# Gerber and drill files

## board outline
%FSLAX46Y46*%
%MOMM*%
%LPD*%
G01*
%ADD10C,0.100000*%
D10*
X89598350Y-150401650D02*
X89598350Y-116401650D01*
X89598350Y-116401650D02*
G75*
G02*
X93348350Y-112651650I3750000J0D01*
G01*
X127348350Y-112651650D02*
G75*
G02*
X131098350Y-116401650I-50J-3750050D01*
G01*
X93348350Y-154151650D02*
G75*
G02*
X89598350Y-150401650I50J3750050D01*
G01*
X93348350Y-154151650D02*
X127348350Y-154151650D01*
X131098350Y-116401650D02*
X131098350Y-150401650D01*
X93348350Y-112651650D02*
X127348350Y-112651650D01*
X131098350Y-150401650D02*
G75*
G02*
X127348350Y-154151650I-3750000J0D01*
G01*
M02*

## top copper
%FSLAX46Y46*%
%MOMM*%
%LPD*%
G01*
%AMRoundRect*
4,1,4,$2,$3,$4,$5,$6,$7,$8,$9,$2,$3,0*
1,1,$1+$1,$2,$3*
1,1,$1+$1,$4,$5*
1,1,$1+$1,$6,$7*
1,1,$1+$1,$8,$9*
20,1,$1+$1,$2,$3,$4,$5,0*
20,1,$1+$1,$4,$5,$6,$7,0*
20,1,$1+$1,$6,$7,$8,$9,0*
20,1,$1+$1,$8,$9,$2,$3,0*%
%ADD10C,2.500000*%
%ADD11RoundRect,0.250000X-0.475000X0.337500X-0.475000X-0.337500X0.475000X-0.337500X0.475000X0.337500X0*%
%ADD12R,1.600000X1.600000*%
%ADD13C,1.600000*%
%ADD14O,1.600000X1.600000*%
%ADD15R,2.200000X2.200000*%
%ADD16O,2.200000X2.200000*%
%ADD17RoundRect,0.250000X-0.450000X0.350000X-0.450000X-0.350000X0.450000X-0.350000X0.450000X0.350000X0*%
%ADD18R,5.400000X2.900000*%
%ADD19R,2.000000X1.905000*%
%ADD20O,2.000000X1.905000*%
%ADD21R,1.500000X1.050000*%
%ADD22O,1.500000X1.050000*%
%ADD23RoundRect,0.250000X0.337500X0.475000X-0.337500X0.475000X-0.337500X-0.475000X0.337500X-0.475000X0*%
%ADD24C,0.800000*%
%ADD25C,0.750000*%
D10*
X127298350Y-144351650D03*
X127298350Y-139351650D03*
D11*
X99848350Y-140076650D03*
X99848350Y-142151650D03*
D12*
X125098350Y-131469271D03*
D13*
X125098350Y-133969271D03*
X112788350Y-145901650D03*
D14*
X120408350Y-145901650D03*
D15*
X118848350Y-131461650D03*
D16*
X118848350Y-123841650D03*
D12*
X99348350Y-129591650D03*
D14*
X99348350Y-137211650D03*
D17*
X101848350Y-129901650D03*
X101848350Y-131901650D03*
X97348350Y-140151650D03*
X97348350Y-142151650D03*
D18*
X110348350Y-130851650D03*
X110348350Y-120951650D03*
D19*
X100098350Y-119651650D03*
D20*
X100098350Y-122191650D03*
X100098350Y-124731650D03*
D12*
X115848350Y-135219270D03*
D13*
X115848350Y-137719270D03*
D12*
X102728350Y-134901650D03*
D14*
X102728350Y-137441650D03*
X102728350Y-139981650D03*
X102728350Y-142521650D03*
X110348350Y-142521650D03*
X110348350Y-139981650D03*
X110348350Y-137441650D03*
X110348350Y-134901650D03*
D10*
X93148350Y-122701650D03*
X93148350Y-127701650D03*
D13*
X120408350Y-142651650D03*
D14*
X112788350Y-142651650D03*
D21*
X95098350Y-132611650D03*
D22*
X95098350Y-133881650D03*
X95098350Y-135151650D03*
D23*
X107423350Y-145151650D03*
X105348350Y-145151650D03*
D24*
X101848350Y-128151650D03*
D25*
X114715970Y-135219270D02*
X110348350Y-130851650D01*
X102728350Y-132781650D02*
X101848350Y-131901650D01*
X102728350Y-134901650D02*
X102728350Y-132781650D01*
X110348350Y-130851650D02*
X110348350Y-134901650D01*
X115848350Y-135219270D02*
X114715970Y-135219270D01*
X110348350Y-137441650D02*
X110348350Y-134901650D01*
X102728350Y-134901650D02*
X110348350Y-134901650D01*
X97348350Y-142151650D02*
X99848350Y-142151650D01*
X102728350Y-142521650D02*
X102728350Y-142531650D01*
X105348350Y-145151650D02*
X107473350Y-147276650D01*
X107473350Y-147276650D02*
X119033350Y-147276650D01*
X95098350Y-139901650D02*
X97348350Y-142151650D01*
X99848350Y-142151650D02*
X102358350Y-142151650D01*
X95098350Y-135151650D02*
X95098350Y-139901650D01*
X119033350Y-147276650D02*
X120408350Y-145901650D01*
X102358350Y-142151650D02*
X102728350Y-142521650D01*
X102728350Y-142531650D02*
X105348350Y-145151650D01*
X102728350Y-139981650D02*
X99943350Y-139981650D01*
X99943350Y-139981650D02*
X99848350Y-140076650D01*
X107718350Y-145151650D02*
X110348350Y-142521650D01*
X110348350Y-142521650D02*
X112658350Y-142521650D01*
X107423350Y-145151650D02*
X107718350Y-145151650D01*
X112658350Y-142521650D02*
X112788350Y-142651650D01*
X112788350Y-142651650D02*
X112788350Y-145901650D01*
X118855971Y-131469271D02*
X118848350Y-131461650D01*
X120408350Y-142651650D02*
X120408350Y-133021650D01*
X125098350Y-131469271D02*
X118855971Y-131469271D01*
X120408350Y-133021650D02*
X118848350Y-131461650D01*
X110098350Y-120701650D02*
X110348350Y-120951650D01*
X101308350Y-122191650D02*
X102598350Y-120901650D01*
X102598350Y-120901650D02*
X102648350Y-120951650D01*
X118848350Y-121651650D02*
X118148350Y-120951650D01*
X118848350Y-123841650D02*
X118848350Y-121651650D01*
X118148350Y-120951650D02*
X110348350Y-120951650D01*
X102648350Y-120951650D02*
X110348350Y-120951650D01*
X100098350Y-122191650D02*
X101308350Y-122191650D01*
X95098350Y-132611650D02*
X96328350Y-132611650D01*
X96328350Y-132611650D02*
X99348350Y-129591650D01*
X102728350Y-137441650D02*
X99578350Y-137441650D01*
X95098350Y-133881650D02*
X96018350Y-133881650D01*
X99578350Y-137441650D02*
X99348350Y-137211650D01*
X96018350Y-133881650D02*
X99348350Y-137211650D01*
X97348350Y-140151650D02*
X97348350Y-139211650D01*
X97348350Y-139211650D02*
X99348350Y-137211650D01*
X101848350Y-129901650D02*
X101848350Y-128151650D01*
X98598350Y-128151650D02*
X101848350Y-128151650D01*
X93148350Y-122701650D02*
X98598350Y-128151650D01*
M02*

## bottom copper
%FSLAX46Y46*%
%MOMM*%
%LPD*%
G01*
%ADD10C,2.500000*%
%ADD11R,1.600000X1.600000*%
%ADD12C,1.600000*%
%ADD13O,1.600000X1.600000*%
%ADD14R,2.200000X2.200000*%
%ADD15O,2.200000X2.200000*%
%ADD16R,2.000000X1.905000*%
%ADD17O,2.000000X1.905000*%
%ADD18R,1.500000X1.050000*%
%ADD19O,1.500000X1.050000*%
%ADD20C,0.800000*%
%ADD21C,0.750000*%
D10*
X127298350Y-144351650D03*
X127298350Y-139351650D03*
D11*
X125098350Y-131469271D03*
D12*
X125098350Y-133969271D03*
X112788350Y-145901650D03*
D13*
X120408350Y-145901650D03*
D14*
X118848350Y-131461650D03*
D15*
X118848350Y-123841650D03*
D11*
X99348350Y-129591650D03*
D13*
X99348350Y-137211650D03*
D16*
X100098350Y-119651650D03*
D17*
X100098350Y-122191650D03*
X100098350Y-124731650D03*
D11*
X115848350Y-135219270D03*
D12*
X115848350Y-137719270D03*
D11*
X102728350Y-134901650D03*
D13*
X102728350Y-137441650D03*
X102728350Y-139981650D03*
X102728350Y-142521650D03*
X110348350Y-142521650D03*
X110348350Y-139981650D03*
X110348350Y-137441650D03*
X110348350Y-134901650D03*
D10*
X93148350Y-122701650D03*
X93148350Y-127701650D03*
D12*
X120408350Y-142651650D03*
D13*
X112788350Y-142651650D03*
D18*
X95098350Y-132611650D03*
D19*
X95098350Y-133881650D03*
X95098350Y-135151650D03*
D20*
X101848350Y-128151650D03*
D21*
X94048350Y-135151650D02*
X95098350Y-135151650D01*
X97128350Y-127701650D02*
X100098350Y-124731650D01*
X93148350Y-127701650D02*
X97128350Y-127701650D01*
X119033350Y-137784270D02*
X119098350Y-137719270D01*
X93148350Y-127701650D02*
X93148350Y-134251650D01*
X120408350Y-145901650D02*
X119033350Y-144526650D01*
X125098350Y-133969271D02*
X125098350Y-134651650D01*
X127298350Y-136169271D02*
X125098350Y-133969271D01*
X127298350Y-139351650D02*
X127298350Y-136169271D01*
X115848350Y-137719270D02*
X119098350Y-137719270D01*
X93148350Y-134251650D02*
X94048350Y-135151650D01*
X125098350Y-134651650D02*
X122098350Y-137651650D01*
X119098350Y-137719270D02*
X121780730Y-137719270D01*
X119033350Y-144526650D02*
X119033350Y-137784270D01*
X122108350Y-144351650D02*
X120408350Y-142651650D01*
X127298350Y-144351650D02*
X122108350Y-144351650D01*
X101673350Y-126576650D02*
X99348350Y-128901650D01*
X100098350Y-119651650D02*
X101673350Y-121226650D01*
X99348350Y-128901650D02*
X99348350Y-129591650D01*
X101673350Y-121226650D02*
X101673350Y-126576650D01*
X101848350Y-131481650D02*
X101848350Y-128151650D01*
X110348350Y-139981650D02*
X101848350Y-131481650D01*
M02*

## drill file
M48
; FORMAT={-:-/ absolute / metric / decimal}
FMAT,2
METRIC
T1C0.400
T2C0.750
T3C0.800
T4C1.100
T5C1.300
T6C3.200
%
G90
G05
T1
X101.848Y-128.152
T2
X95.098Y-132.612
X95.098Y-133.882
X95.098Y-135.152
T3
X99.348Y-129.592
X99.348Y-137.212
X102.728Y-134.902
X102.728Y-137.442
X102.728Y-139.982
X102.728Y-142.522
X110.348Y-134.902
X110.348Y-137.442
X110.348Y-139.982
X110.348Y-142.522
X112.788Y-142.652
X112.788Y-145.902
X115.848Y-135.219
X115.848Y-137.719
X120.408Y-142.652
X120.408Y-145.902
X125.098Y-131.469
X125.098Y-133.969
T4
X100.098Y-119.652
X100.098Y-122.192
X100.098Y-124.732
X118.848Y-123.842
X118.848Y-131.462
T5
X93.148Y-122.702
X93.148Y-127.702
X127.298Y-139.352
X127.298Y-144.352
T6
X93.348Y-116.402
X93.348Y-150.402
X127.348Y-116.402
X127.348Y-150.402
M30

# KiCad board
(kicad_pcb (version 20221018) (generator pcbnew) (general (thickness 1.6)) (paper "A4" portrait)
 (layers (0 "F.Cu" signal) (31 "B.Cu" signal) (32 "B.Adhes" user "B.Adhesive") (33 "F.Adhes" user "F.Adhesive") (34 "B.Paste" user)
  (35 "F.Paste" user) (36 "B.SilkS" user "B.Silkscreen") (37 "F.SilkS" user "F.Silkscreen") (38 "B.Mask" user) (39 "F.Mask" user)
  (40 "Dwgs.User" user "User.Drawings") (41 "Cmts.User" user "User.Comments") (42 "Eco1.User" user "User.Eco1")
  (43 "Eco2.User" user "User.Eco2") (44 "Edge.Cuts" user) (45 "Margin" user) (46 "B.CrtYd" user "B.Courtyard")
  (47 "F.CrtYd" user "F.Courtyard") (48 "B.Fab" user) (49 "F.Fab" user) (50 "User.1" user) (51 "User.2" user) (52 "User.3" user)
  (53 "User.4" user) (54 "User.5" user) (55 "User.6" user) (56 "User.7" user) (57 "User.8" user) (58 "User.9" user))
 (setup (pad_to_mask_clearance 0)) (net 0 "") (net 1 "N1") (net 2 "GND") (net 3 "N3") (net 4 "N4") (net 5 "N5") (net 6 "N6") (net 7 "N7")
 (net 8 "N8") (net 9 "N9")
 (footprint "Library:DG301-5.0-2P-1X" (layer "F.Cu") (at 127.29835 141.85165 90)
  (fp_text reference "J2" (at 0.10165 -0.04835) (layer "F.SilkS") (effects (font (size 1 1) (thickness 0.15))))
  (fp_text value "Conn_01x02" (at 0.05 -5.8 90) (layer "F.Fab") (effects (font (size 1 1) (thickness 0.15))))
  (pad "1" thru_hole circle (at -2.5 0 90) (size 2.5 2.5) (drill 1.3) (layers "*.Cu" "*.Mask") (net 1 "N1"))
  (pad "2" thru_hole circle (at 2.5 0 90) (size 2.5 2.5) (drill 1.3) (layers "*.Cu" "*.Mask") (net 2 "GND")))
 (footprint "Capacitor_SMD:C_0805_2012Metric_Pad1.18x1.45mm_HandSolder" (layer "F.Cu") (at 99.84835 141.11415 -90)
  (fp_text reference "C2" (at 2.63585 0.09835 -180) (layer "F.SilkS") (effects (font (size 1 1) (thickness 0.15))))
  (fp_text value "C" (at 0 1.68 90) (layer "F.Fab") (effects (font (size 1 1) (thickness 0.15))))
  (pad "1" smd roundrect (at -1.0375 0 270) (size 1.175 1.45) (layers "F.Cu" "F.Paste" "F.Mask") (roundrect_rratio 0.212766) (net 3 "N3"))
  (pad "2" smd roundrect (at 1.0375 0 270) (size 1.175 1.45) (layers "F.Cu" "F.Paste" "F.Mask") (roundrect_rratio 0.212766) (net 2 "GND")))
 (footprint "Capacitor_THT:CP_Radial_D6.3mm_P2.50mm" (layer "F.Cu") (at 125.09835 131.469271 -90)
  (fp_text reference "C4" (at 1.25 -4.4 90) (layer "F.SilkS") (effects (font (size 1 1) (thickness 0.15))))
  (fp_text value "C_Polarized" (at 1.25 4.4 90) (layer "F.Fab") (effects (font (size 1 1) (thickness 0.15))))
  (pad "1" thru_hole rect (at 0 0 270) (size 1.6 1.6) (drill 0.8) (layers "*.Cu" "*.Mask") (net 1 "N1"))
  (pad "2" thru_hole circle (at 2.5 0 270) (size 1.6 1.6) (drill 0.8) (layers "*.Cu" "*.Mask") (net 2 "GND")))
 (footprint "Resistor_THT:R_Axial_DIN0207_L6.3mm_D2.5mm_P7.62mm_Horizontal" (layer "F.Cu") (at 112.78835 145.90165)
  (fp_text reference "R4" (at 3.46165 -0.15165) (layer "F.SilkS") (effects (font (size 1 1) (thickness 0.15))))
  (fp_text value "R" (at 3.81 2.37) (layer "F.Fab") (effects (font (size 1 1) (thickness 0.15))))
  (pad "1" thru_hole circle (at 0 0) (size 1.6 1.6) (drill 0.8) (layers "*.Cu" "*.Mask") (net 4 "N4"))
  (pad "2" thru_hole oval (at 7.62 0) (size 1.6 1.6) (drill 0.8) (layers "*.Cu" "*.Mask") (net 2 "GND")))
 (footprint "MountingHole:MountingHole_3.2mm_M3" (layer "F.Cu") (at 93.34835 116.40165)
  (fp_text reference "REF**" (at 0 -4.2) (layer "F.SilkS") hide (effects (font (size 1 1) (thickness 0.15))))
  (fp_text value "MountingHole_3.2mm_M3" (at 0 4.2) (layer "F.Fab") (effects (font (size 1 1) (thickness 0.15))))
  (pad "" np_thru_hole circle (at 0 0) (size 3.2 3.2) (drill 3.2) (layers "*.Cu" "*.Mask")))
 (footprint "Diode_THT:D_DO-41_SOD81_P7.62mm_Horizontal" (layer "F.Cu") (at 118.84835 131.46165 90)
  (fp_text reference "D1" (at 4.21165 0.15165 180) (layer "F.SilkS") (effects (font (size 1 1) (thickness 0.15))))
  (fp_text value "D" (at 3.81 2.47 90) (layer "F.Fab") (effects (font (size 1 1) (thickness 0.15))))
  (pad "1" thru_hole rect (at 0 0 90) (size 2.2 2.2) (drill 1.1) (layers "*.Cu" "*.Mask") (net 1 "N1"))
  (pad "2" thru_hole oval (at 7.62 0 90) (size 2.2 2.2) (drill 1.1) (layers "*.Cu" "*.Mask") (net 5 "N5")))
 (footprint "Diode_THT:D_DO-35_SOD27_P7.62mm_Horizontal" (layer "F.Cu") (at 99.34835 129.59165 -90)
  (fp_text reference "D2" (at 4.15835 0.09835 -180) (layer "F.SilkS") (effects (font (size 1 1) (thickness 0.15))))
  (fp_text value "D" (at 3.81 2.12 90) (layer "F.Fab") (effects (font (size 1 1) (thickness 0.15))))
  (pad "1" thru_hole rect (at 0 0 270) (size 1.6 1.6) (drill 0.8) (layers "*.Cu" "*.Mask") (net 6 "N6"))
  (pad "2" thru_hole oval (at 7.62 0 270) (size 1.6 1.6) (drill 0.8) (layers "*.Cu" "*.Mask") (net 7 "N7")))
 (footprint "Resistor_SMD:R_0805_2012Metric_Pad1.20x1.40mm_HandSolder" (layer "F.Cu") (at 101.84835 130.90165 -90)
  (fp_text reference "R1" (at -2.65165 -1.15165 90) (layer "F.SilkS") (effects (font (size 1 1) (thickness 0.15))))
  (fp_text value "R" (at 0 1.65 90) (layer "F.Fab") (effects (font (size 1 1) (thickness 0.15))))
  (pad "1" smd roundrect (at -1 0 270) (size 1.2 1.4) (layers "F.Cu" "F.Paste" "F.Mask") (roundrect_rratio 0.208333) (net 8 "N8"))
  (pad "2" smd roundrect (at 1 0 270) (size 1.2 1.4) (layers "F.Cu" "F.Paste" "F.Mask") (roundrect_rratio 0.208333) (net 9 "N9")))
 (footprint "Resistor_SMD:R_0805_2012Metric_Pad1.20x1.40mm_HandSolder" (layer "F.Cu") (at 97.34835 141.15165 -90)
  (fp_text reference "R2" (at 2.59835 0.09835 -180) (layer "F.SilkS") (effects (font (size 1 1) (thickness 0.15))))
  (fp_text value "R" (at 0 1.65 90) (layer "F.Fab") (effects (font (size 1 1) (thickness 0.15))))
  (pad "1" smd roundrect (at -1 0 270) (size 1.2 1.4) (layers "F.Cu" "F.Paste" "F.Mask") (roundrect_rratio 0.208333) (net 7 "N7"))
  (pad "2" smd roundrect (at 1 0 270) (size 1.2 1.4) (layers "F.Cu" "F.Paste" "F.Mask") (roundrect_rratio 0.208333) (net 2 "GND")))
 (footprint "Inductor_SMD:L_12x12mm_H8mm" (layer "F.Cu") (at 110.34835 125.90165 90)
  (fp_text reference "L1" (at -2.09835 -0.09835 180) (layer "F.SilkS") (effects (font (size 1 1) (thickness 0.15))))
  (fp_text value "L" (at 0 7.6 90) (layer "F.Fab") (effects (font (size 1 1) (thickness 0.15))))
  (pad "1" smd rect (at -4.95 0 90) (size 2.9 5.4) (layers "F.Cu" "F.Paste" "F.Mask") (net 9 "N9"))
  (pad "2" smd rect (at 4.95 0 90) (size 2.9 5.4) (layers "F.Cu" "F.Paste" "F.Mask") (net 5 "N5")))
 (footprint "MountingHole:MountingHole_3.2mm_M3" (layer "F.Cu") (at 127.34835 150.40165)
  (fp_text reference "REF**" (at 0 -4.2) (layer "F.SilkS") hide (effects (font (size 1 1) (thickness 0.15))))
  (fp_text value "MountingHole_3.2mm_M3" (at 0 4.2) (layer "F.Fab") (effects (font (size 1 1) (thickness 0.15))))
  (pad "" np_thru_hole circle (at 0 0) (size 3.2 3.2) (drill 3.2) (layers "*.Cu" "*.Mask")))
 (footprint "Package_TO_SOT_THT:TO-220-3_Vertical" (layer "F.Cu") (at 100.09835 119.65165 -90)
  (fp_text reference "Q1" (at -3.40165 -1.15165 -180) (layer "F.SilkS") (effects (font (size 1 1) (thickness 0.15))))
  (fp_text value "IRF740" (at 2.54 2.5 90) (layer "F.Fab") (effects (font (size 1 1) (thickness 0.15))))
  (pad "1" thru_hole rect (at 0 0 270) (size 1.905 2) (drill 1.1) (layers "*.Cu" "*.Mask") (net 6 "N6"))
  (pad "2" thru_hole oval (at 2.54 0 270) (size 1.905 2) (drill 1.1) (layers "*.Cu" "*.Mask") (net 5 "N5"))
  (pad "3" thru_hole oval (at 5.08 0 270) (size 1.905 2) (drill 1.1) (layers "*.Cu" "*.Mask") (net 2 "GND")))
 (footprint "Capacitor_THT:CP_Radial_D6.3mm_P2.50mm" (layer "F.Cu") (at 115.84835 135.21927 -90)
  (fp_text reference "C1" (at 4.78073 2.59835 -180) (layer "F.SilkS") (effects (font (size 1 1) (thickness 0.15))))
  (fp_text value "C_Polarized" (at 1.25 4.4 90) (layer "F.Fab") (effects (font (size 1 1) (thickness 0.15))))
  (pad "1" thru_hole rect (at 0 0 270) (size 1.6 1.6) (drill 0.8) (layers "*.Cu" "*.Mask") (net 9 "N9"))
  (pad "2" thru_hole circle (at 2.5 0 270) (size 1.6 1.6) (drill 0.8) (layers "*.Cu" "*.Mask") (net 2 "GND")))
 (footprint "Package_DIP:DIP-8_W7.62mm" (layer "F.Cu") (at 102.72835 134.90165)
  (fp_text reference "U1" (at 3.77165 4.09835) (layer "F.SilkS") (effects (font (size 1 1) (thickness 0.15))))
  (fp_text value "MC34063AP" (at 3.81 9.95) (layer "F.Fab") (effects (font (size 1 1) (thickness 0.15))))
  (pad "1" thru_hole rect (at 0 0) (size 1.6 1.6) (drill 0.8) (layers "*.Cu" "*.Mask") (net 9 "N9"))
  (pad "2" thru_hole oval (at 0 2.54) (size 1.6 1.6) (drill 0.8) (layers "*.Cu" "*.Mask") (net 7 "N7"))
  (pad "3" thru_hole oval (at 0 5.08) (size 1.6 1.6) (drill 0.8) (layers "*.Cu" "*.Mask") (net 3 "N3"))
  (pad "4" thru_hole oval (at 0 7.62) (size 1.6 1.6) (drill 0.8) (layers "*.Cu" "*.Mask") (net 2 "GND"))
  (pad "5" thru_hole oval (at 7.62 7.62) (size 1.6 1.6) (drill 0.8) (layers "*.Cu" "*.Mask") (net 4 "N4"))
  (pad "6" thru_hole oval (at 7.62 5.08) (size 1.6 1.6) (drill 0.8) (layers "*.Cu" "*.Mask") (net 8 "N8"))
  (pad "7" thru_hole oval (at 7.62 2.54) (size 1.6 1.6) (drill 0.8) (layers "*.Cu" "*.Mask") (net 9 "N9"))
  (pad "8" thru_hole oval (at 7.62 0) (size 1.6 1.6) (drill 0.8) (layers "*.Cu" "*.Mask") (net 9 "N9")))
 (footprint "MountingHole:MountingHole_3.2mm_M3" (layer "F.Cu") (at 93.34835 150.40165)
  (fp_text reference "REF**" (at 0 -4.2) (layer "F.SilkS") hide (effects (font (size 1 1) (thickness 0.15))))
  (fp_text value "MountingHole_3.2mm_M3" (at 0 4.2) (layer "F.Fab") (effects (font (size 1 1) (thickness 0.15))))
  (pad "" np_thru_hole circle (at 0 0) (size 3.2 3.2) (drill 3.2) (layers "*.Cu" "*.Mask")))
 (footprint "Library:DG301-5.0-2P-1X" (layer "F.Cu") (at 93.14835 125.20165 -90)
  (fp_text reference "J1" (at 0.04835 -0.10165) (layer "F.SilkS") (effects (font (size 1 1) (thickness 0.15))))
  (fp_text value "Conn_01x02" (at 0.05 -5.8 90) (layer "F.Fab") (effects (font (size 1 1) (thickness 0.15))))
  (pad "1" thru_hole circle (at -2.5 0 270) (size 2.5 2.5) (drill 1.3) (layers "*.Cu" "*.Mask") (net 8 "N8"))
  (pad "2" thru_hole circle (at 2.5 0 270) (size 2.5 2.5) (drill 1.3) (layers "*.Cu" "*.Mask") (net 2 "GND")))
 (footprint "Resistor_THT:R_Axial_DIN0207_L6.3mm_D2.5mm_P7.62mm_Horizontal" (layer "F.Cu") (at 120.40835 142.65165 180)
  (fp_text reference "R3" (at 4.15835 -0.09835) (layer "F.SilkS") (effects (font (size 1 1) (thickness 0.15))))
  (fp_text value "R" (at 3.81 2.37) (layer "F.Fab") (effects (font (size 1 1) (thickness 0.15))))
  (pad "1" thru_hole circle (at 0 0 180) (size 1.6 1.6) (drill 0.8) (layers "*.Cu" "*.Mask") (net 1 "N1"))
  (pad "2" thru_hole oval (at 7.62 0 180) (size 1.6 1.6) (drill 0.8) (layers "*.Cu" "*.Mask") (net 4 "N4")))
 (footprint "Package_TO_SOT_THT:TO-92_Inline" (layer "F.Cu") (at 95.09835 132.61165 -90)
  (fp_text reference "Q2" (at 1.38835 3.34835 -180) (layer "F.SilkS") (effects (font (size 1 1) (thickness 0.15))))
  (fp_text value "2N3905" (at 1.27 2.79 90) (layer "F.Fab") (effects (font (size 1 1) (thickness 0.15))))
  (pad "1" thru_hole rect (at 0 0 270) (size 1.05 1.5) (drill 0.75) (layers "*.Cu" "*.Mask") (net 6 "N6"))
  (pad "2" thru_hole oval (at 1.27 0 270) (size 1.05 1.5) (drill 0.75) (layers "*.Cu" "*.Mask") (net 7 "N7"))
  (pad "3" thru_hole oval (at 2.54 0 270) (size 1.05 1.5) (drill 0.75) (layers "*.Cu" "*.Mask") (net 2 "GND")))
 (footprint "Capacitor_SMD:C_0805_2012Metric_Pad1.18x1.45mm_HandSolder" (layer "F.Cu") (at 106.38585 145.15165 180)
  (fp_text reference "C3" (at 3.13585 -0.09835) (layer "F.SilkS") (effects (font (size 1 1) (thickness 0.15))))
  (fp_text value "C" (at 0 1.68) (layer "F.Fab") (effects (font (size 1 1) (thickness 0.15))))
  (pad "1" smd roundrect (at -1.0375 0 180) (size 1.175 1.45) (layers "F.Cu" "F.Paste" "F.Mask") (roundrect_rratio 0.212766) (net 4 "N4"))
  (pad "2" smd roundrect (at 1.0375 0 180) (size 1.175 1.45) (layers "F.Cu" "F.Paste" "F.Mask") (roundrect_rratio 0.212766) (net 2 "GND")))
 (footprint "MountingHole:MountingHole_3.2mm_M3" (layer "F.Cu") (at 127.34835 116.40165)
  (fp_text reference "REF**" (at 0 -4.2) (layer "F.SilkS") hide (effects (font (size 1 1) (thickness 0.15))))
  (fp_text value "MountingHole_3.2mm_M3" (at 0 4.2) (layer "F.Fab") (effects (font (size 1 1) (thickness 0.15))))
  (pad "" np_thru_hole circle (at 0 0) (size 3.2 3.2) (drill 3.2) (layers "*.Cu" "*.Mask")))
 (gr_line (start 89.59835 150.40165) (end 89.59835 116.40165) (stroke (width 0.1) (type default)) (layer "Edge.Cuts"))
 (gr_arc (start 89.59835 116.40165) (mid 90.6967 113.75) (end 93.34835 112.65165) (stroke (width 0.1) (type default)) (layer "Edge.Cuts"))
 (gr_arc (start 127.34835 112.65165) (mid 130 113.75) (end 131.09835 116.40165) (stroke (width 0.1) (type default)) (layer "Edge.Cuts"))
 (gr_arc (start 93.34835 154.15165) (mid 90.6967 153.0533) (end 89.59835 150.40165) (stroke (width 0.1) (type default)) (layer "Edge.Cuts"))
 (gr_line (start 93.34835 154.15165) (end 127.34835 154.15165) (stroke (width 0.1) (type default)) (layer "Edge.Cuts"))
 (gr_line (start 131.09835 116.40165) (end 131.09835 150.40165) (stroke (width 0.1) (type default)) (layer "Edge.Cuts"))
 (gr_line (start 93.34835 112.65165) (end 127.34835 112.65165) (stroke (width 0.1) (type default)) (layer "Edge.Cuts"))
 (gr_arc (start 131.09835 150.40165) (mid 130 153.0533) (end 127.34835 154.15165) (stroke (width 0.1) (type default)) (layer "Edge.Cuts"))
 (segment (start 114.71597 135.21927) (end 110.34835 130.85165) (width 0.75) (layer "F.Cu") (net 9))
 (segment (start 102.72835 132.78165) (end 101.84835 131.90165) (width 0.75) (layer "F.Cu") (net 9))
 (segment (start 102.72835 134.90165) (end 102.72835 132.78165) (width 0.75) (layer "F.Cu") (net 9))
 (segment (start 110.34835 130.85165) (end 110.34835 134.90165) (width 0.75) (layer "F.Cu") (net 9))
 (segment (start 115.84835 135.21927) (end 114.71597 135.21927) (width 0.75) (layer "F.Cu") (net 9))
 (segment (start 110.34835 137.44165) (end 110.34835 134.90165) (width 0.75) (layer "F.Cu") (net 9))
 (segment (start 102.72835 134.90165) (end 110.34835 134.90165) (width 0.75) (layer "F.Cu") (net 9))
 (segment (start 97.34835 142.15165) (end 99.84835 142.15165) (width 0.75) (layer "F.Cu") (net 2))
 (segment (start 102.72835 142.52165) (end 102.72835 142.53165) (width 0.75) (layer "F.Cu") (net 2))
 (segment (start 105.34835 145.15165) (end 107.47335 147.27665) (width 0.75) (layer "F.Cu") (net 2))
 (segment (start 107.47335 147.27665) (end 119.03335 147.27665) (width 0.75) (layer "F.Cu") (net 2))
 (segment (start 95.09835 139.90165) (end 97.34835 142.15165) (width 0.75) (layer "F.Cu") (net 2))
 (segment (start 99.84835 142.15165) (end 102.35835 142.15165) (width 0.75) (layer "F.Cu") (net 2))
 (segment (start 95.09835 135.15165) (end 95.09835 139.90165) (width 0.75) (layer "F.Cu") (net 2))
 (segment (start 119.03335 147.27665) (end 120.40835 145.90165) (width 0.75) (layer "F.Cu") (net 2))
 (segment (start 102.35835 142.15165) (end 102.72835 142.52165) (width 0.75) (layer "F.Cu") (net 2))
 (segment (start 102.72835 142.53165) (end 105.34835 145.15165) (width 0.75) (layer "F.Cu") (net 2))
 (segment (start 94.04835 135.15165) (end 95.09835 135.15165) (width 0.75) (layer "B.Cu") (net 2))
 (segment (start 97.12835 127.70165) (end 100.09835 124.73165) (width 0.75) (layer "B.Cu") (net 2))
 (segment (start 93.14835 127.70165) (end 97.12835 127.70165) (width 0.75) (layer "B.Cu") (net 2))
 (segment (start 119.03335 137.78427) (end 119.09835 137.71927) (width 0.75) (layer "B.Cu") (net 2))
 (segment (start 93.14835 127.70165) (end 93.14835 134.25165) (width 0.75) (layer "B.Cu") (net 2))
 (segment (start 120.40835 145.90165) (end 119.03335 144.52665) (width 0.75) (layer "B.Cu") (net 2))
 (segment (start 125.09835 133.969271) (end 125.09835 134.65165) (width 0.75) (layer "B.Cu") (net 2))
 (segment (start 127.29835 136.169271) (end 125.09835 133.969271) (width 0.75) (layer "B.Cu") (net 2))
 (segment (start 127.29835 139.35165) (end 127.29835 136.169271) (width 0.75) (layer "B.Cu") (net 2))
 (segment (start 115.84835 137.71927) (end 119.09835 137.71927) (width 0.75) (layer "B.Cu") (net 2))
 (segment (start 93.14835 134.25165) (end 94.04835 135.15165) (width 0.75) (layer "B.Cu") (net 2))
 (segment (start 125.09835 134.65165) (end 122.09835 137.65165) (width 0.75) (layer "B.Cu") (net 2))
 (segment (start 119.09835 137.71927) (end 121.78073 137.71927) (width 0.75) (layer "B.Cu") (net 2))
 (segment (start 119.03335 144.52665) (end 119.03335 137.78427) (width 0.75) (layer "B.Cu") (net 2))
 (segment (start 102.72835 139.98165) (end 99.94335 139.98165) (width 0.75) (layer "F.Cu") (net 3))
 (segment (start 99.94335 139.98165) (end 99.84835 140.07665) (width 0.75) (layer "F.Cu") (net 3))
 (segment (start 107.71835 145.15165) (end 110.34835 142.52165) (width 0.75) (layer "F.Cu") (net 4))
 (segment (start 110.34835 142.52165) (end 112.65835 142.52165) (width 0.75) (layer "F.Cu") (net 4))
 (segment (start 107.42335 145.15165) (end 107.71835 145.15165) (width 0.75) (layer "F.Cu") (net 4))
 (segment (start 112.65835 142.52165) (end 112.78835 142.65165) (width 0.75) (layer "F.Cu") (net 4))
 (segment (start 112.78835 142.65165) (end 112.78835 145.90165) (width 0.75) (layer "F.Cu") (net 4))
 (segment (start 118.855971 131.469271) (end 118.84835 131.46165) (width 0.75) (layer "F.Cu") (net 1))
 (segment (start 120.40835 142.65165) (end 120.40835 133.02165) (width 0.75) (layer "F.Cu") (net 1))
 (segment (start 125.09835 131.469271) (end 118.855971 131.469271) (width 0.75) (layer "F.Cu") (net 1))
 (segment (start 120.40835 133.02165) (end 118.84835 131.46165) (width 0.75) (layer "F.Cu") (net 1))
 (segment (start 122.10835 144.35165) (end 120.40835 142.65165) (width 0.75) (layer "B.Cu") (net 1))
 (segment (start 127.29835 144.35165) (end 122.10835 144.35165) (width 0.75) (layer "B.Cu") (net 1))
 (segment (start 110.09835 120.70165) (end 110.34835 120.95165) (width 0.75) (layer "F.Cu") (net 5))
 (segment (start 101.30835 122.19165) (end 102.59835 120.90165) (width 0.75) (layer "F.Cu") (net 5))
 (segment (start 102.59835 120.90165) (end 102.64835 120.95165) (width 0.75) (layer "F.Cu") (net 5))
 (segment (start 118.84835 121.65165) (end 118.14835 120.95165) (width 0.75) (layer "F.Cu") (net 5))
 (segment (start 118.84835 123.84165) (end 118.84835 121.65165) (width 0.75) (layer "F.Cu") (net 5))
 (segment (start 118.14835 120.95165) (end 110.34835 120.95165) (width 0.75) (layer "F.Cu") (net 5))
 (segment (start 102.64835 120.95165) (end 110.34835 120.95165) (width 0.75) (layer "F.Cu") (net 5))
 (segment (start 100.09835 122.19165) (end 101.30835 122.19165) (width 0.75) (layer "F.Cu") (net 5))
 (segment (start 95.09835 132.61165) (end 96.32835 132.61165) (width 0.75) (layer "F.Cu") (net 6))
 (segment (start 96.32835 132.61165) (end 99.34835 129.59165) (width 0.75) (layer "F.Cu") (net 6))
 (segment (start 101.67335 126.57665) (end 99.34835 128.90165) (width 0.75) (layer "B.Cu") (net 6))
 (segment (start 100.09835 119.65165) (end 101.67335 121.22665) (width 0.75) (layer "B.Cu") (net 6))
 (segment (start 99.34835 128.90165) (end 99.34835 129.59165) (width 0.75) (layer "B.Cu") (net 6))
 (segment (start 101.67335 121.22665) (end 101.67335 126.57665) (width 0.75) (layer "B.Cu") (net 6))
 (segment (start 102.72835 137.44165) (end 99.57835 137.44165) (width 0.75) (layer "F.Cu") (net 7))
 (segment (start 95.09835 133.88165) (end 96.01835 133.88165) (width 0.75) (layer "F.Cu") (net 7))
 (segment (start 99.57835 137.44165) (end 99.34835 137.21165) (width 0.75) (layer "F.Cu") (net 7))
 (segment (start 96.01835 133.88165) (end 99.34835 137.21165) (width 0.75) (layer "F.Cu") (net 7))
 (segment (start 97.34835 140.15165) (end 97.34835 139.21165) (width 0.75) (layer "F.Cu") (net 7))
 (segment (start 97.34835 139.21165) (end 99.34835 137.21165) (width 0.75) (layer "F.Cu") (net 7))
 (segment (start 101.84835 129.90165) (end 101.84835 128.15165) (width 0.75) (layer "F.Cu") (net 8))
 (segment (start 98.59835 128.15165) (end 101.84835 128.15165) (width 0.75) (layer "F.Cu") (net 8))
 (segment (start 93.14835 122.70165) (end 98.59835 128.15165) (width 0.75) (layer "F.Cu") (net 8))
 (via (at 101.84835 128.15165) (size 0.8) (drill 0.4) (layers "F.Cu" "B.Cu") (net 8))
 (segment (start 101.84835 131.48165) (end 101.84835 128.15165) (width 0.75) (layer "B.Cu") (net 8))
 (segment (start 110.34835 139.98165) (end 101.84835 131.48165) (width 0.75) (layer "B.Cu") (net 8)))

